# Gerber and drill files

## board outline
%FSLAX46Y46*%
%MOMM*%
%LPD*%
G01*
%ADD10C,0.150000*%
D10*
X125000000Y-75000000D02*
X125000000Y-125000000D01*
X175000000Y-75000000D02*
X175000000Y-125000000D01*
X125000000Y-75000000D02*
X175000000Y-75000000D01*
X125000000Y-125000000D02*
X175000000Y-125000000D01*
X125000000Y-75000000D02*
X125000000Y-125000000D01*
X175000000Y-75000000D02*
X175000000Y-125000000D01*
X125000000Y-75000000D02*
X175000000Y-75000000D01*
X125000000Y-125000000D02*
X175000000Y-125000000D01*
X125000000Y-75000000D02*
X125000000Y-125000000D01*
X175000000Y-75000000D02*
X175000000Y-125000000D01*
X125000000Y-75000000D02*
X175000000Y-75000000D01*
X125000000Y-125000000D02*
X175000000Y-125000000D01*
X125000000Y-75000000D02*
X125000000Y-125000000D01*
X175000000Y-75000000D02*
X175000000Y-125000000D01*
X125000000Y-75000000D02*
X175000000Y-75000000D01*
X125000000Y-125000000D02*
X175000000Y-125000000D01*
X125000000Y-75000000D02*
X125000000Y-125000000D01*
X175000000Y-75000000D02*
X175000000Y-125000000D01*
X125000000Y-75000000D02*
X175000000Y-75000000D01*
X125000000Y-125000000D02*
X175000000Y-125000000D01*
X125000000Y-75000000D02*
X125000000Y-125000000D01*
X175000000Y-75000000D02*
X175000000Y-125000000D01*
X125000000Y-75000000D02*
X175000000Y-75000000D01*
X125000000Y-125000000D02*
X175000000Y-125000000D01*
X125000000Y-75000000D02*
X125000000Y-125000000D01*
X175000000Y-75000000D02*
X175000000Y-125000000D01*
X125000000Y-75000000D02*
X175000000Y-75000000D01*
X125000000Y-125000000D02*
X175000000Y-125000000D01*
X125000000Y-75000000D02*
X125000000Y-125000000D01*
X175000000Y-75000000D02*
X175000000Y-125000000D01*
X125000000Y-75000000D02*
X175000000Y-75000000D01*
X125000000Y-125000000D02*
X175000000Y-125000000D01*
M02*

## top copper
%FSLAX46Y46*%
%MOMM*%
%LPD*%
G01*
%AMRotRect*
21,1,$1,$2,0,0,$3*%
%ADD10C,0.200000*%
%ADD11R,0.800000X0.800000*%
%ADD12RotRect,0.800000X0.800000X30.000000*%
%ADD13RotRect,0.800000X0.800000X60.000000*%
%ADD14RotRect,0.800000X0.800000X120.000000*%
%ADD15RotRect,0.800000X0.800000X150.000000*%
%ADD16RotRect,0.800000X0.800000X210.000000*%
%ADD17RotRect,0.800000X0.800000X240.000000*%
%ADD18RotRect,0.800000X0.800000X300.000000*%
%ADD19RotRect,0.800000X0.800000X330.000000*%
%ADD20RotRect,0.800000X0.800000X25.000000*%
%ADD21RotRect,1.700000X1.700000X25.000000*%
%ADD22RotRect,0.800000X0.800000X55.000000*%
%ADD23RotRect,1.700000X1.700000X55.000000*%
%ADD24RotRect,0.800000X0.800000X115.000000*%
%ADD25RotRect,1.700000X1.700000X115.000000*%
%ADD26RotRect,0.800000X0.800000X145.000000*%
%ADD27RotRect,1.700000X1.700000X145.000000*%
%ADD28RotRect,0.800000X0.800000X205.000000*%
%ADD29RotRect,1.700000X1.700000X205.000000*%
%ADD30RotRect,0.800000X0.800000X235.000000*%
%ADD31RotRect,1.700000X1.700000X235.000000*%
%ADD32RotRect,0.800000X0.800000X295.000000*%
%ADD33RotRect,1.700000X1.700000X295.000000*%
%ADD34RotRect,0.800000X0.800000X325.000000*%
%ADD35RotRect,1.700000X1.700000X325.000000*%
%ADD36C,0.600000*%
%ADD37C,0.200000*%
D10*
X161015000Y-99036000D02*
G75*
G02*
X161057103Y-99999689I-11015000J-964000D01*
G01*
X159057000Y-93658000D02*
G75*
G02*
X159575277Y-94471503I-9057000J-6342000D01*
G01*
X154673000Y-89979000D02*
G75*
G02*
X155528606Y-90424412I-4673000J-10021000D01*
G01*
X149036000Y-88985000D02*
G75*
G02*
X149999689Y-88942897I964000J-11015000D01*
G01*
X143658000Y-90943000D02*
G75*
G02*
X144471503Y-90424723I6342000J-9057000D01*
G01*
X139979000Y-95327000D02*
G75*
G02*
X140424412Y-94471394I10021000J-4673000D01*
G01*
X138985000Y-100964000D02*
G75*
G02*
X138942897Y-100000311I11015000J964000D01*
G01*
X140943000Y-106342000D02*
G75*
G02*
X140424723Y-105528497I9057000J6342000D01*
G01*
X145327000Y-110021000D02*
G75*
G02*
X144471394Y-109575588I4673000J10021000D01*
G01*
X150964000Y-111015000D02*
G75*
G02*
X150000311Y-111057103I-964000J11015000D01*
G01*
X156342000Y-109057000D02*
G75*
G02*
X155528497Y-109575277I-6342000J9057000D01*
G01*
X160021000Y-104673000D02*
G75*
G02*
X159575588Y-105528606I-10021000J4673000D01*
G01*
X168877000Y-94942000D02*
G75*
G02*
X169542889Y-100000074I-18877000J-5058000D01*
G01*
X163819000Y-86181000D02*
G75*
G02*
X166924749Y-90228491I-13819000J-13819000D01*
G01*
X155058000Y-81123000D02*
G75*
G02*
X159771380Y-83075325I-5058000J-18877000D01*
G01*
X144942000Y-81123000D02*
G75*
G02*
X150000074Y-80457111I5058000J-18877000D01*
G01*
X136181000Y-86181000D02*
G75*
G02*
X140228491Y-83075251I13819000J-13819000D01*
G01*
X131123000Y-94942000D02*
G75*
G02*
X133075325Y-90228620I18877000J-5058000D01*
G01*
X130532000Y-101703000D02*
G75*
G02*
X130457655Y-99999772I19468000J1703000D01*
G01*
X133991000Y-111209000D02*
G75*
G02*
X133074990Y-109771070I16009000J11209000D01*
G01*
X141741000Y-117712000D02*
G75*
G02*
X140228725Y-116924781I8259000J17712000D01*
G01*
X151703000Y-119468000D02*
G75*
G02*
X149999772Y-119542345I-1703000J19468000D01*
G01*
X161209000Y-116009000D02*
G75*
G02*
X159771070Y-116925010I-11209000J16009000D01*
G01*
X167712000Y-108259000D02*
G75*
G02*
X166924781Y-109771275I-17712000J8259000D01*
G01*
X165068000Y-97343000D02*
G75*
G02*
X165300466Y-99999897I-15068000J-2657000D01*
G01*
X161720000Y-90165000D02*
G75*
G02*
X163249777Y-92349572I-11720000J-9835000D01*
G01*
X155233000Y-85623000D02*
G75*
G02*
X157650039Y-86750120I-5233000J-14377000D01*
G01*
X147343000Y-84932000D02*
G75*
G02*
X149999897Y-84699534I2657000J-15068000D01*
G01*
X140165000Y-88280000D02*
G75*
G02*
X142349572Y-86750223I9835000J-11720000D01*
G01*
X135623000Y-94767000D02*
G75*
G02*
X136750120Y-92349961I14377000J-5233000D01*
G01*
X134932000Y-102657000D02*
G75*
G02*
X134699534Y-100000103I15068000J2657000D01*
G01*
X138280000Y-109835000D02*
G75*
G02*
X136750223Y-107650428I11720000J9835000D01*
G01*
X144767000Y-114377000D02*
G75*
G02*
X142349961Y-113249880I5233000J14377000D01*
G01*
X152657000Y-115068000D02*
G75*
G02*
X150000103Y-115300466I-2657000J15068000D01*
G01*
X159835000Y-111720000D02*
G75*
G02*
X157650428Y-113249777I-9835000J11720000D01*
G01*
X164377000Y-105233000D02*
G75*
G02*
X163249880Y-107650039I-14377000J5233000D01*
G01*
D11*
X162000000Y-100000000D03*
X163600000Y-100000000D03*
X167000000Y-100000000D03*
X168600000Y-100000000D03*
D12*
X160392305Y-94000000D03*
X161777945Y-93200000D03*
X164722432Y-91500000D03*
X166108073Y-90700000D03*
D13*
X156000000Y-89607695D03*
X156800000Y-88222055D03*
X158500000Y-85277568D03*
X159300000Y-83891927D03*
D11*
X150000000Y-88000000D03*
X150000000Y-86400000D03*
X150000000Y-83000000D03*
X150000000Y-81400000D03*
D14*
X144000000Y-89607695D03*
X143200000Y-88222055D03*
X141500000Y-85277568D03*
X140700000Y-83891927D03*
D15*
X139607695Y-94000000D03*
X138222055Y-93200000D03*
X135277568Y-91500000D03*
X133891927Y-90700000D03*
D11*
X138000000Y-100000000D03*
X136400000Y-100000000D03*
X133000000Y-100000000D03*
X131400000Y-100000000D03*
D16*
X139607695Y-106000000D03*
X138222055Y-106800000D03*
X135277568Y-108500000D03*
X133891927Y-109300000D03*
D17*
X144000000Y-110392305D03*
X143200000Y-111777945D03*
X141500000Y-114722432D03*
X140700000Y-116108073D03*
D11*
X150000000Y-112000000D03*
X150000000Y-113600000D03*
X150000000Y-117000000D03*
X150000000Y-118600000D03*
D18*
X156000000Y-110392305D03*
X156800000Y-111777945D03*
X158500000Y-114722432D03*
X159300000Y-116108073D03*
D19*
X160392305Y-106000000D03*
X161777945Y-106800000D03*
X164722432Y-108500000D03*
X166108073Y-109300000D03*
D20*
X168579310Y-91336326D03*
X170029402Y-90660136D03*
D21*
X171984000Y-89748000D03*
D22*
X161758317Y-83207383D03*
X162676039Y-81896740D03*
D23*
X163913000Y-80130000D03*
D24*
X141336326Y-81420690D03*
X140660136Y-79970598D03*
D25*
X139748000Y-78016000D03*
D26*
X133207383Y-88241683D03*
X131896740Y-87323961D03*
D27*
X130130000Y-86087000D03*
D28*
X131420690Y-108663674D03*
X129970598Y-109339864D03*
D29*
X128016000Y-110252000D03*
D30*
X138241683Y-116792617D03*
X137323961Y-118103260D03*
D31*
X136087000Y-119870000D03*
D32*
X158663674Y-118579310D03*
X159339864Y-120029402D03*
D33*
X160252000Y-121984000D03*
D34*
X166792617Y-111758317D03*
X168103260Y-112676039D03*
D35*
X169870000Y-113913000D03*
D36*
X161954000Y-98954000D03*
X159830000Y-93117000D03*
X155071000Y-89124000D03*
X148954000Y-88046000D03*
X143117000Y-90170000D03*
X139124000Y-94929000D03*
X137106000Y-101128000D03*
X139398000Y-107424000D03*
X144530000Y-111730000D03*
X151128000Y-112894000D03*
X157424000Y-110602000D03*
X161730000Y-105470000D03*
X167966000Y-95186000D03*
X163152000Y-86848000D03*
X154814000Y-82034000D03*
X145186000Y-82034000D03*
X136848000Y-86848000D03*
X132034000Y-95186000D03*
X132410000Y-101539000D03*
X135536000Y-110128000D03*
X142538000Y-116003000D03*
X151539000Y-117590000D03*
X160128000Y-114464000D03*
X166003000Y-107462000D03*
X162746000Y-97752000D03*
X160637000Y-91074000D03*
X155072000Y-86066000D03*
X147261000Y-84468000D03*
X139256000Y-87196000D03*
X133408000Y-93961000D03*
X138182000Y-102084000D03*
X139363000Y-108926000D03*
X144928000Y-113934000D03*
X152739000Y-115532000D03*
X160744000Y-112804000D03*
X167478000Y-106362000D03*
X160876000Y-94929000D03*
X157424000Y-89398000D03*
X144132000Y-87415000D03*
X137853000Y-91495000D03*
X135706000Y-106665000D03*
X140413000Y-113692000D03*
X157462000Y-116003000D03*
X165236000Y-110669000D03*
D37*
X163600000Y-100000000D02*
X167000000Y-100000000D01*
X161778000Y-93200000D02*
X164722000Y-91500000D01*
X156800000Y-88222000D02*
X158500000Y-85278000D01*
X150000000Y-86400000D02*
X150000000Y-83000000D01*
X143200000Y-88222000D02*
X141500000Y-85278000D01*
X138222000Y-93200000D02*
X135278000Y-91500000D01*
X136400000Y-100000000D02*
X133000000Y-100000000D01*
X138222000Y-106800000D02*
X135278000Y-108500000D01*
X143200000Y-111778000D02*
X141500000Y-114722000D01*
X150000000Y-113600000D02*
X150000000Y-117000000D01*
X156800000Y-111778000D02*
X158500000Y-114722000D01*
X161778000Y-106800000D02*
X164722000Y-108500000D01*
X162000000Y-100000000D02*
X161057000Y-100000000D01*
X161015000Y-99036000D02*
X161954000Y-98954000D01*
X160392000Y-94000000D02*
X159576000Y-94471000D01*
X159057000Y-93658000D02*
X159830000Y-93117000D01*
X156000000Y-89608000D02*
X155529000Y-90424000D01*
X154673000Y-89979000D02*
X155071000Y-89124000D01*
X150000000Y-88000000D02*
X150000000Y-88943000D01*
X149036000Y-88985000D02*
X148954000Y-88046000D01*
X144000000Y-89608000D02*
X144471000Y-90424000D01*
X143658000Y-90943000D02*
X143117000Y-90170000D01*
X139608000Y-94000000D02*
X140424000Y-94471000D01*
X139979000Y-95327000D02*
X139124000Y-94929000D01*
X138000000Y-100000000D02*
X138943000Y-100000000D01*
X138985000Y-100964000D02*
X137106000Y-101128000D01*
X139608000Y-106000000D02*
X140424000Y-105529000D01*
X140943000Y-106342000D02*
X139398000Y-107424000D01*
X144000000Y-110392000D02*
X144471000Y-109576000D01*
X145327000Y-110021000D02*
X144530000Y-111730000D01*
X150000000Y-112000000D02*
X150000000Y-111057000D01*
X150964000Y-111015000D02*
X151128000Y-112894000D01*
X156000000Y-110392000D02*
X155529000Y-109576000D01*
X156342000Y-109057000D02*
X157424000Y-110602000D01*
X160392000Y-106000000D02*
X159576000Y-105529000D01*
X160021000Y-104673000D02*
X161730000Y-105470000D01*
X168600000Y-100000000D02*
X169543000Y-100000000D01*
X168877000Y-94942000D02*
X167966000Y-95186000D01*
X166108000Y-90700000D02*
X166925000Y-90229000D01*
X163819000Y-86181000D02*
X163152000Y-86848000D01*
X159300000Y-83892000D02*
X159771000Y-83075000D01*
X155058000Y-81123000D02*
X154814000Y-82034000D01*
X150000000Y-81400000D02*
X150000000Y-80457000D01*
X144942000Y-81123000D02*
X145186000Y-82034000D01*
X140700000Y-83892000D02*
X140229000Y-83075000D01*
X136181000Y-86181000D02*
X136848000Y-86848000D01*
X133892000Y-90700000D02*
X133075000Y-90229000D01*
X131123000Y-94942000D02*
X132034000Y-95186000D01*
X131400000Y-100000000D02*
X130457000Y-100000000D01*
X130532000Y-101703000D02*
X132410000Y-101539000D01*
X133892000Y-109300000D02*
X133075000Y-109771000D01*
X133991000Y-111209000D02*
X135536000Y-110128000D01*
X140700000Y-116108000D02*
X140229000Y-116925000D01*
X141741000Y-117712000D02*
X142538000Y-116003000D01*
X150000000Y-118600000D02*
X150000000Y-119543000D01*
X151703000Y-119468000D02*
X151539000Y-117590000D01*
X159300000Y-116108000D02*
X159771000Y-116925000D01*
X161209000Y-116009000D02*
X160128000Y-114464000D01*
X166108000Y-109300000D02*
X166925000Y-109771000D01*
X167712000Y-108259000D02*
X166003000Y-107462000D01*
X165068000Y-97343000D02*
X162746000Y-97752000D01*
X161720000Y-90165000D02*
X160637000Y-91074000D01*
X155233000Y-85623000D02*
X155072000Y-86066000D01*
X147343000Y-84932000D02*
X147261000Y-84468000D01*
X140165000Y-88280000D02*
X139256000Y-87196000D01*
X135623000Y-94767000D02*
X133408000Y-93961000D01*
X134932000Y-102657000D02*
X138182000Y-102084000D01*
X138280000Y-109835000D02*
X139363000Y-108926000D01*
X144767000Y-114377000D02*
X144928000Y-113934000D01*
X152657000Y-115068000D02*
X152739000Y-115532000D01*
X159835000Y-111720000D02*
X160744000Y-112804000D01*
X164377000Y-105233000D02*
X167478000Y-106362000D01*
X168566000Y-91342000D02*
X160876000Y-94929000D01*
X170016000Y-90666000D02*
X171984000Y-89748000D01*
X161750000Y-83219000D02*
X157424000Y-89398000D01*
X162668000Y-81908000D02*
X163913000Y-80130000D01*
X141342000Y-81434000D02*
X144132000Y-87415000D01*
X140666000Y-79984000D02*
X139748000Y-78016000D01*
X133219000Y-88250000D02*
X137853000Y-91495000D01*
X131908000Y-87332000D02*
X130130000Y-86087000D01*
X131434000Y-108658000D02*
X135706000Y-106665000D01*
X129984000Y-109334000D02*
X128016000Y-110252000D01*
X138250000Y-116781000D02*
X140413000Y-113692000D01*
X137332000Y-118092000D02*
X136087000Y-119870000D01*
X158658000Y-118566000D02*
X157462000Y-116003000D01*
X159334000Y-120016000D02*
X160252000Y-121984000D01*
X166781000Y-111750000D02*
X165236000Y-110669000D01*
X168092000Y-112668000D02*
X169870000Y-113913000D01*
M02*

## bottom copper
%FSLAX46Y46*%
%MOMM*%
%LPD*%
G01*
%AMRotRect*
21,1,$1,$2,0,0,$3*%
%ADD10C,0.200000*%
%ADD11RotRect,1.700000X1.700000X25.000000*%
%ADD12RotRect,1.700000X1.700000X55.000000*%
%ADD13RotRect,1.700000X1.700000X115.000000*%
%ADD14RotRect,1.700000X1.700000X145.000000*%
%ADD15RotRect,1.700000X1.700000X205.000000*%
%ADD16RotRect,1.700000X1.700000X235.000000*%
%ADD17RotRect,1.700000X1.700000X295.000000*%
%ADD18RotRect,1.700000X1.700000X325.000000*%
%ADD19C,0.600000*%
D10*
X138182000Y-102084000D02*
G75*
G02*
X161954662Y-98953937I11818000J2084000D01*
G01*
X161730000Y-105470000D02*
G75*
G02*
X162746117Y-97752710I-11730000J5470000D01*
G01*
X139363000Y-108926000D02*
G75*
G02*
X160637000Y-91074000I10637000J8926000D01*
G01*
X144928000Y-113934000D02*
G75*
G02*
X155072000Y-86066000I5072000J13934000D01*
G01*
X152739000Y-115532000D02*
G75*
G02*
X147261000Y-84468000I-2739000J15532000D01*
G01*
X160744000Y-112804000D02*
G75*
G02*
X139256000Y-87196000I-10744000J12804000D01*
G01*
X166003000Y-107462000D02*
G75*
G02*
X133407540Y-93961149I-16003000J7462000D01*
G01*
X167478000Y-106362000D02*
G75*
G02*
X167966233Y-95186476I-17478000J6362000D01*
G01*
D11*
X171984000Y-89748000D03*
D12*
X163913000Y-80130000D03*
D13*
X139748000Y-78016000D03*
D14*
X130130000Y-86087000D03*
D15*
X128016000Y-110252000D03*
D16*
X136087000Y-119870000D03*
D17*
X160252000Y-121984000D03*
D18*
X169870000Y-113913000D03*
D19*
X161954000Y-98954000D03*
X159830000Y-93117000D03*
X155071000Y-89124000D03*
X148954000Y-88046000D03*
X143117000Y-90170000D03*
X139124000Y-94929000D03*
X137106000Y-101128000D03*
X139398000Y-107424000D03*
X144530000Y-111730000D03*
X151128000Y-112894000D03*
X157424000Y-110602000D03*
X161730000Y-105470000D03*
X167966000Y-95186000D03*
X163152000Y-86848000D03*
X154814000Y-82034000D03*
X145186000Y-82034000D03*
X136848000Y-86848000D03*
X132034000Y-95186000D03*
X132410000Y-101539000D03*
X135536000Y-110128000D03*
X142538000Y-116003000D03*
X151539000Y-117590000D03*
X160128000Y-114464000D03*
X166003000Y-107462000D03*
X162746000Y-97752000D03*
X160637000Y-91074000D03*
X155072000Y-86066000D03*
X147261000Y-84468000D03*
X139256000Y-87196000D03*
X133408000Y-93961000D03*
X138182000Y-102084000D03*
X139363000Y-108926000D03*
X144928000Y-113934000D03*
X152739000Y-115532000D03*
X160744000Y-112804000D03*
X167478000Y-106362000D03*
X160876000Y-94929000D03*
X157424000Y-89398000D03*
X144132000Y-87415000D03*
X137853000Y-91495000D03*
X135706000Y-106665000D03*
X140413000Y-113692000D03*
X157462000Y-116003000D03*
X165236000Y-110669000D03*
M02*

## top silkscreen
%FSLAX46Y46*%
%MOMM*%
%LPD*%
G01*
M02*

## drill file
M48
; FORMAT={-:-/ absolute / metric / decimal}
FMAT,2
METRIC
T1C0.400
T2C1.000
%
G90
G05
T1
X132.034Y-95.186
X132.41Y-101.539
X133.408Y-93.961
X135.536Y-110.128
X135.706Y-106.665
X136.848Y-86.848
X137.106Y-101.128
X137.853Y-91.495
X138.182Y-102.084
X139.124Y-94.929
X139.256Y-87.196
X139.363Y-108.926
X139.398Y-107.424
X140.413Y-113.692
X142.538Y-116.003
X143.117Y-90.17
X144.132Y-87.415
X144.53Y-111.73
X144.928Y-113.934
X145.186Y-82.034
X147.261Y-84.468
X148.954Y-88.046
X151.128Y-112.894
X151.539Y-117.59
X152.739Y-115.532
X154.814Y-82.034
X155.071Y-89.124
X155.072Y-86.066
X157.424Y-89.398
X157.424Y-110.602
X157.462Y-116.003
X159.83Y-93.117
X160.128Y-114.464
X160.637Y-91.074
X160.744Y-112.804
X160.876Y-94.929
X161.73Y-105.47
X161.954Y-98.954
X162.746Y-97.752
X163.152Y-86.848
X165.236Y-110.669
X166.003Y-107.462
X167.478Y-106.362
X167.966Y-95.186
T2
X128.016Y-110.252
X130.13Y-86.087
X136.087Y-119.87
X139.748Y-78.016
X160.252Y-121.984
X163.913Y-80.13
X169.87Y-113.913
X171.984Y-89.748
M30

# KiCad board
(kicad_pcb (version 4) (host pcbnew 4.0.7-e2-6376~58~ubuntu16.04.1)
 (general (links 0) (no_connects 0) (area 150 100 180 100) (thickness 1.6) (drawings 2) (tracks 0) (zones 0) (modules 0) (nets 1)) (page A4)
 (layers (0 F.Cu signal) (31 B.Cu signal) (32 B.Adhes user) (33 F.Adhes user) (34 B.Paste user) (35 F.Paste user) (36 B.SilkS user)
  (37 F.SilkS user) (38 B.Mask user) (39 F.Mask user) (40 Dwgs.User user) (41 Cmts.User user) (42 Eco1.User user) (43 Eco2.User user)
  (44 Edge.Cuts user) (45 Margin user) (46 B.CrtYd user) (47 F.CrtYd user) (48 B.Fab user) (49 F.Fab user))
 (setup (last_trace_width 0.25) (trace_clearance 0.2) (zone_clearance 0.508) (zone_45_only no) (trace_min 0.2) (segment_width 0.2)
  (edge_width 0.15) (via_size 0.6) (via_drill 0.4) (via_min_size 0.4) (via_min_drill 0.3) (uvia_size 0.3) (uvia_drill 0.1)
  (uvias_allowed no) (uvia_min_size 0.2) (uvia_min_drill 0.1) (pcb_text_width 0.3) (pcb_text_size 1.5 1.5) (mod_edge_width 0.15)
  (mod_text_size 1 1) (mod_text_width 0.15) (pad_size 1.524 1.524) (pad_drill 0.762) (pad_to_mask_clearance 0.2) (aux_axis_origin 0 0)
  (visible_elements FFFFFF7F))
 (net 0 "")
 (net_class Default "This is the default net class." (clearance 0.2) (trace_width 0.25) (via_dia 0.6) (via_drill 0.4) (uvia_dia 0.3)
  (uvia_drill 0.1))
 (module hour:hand (layer F.Cu) (at 150 100 0.0)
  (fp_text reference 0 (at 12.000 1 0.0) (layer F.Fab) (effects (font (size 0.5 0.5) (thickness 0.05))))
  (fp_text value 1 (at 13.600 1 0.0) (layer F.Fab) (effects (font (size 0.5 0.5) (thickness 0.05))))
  (pad 1 smd rect (at 12.0 0 0.0) (size 0.8 0.8) (layers F.Cu F.Paste F.Mask))
  (pad 2 smd rect (at 13.6 0 0.0) (size 0.8 0.8) (layers F.Cu F.Paste F.Mask)))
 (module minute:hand (layer F.Cu) (at 150 100 0.0)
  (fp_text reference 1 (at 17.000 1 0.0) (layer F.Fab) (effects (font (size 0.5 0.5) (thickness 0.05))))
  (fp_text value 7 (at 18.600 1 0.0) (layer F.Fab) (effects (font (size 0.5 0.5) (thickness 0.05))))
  (pad 1 smd rect (at 17.0 0 0.0) (size 0.8 0.8) (layers F.Cu F.Paste F.Mask))
  (pad 2 smd rect (at 18.6 0 0.0) (size 0.8 0.8) (layers F.Cu F.Paste F.Mask)))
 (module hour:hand (layer F.Cu) (at 150 100 30.0)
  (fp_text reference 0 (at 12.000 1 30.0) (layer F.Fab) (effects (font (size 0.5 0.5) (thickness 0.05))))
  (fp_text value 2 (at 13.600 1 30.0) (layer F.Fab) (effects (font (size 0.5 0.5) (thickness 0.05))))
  (pad 1 smd rect (at 12.0 0 30.0) (size 0.8 0.8) (layers F.Cu F.Paste F.Mask))
  (pad 2 smd rect (at 13.6 0 30.0) (size 0.8 0.8) (layers F.Cu F.Paste F.Mask)))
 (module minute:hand (layer F.Cu) (at 150 100 30.0)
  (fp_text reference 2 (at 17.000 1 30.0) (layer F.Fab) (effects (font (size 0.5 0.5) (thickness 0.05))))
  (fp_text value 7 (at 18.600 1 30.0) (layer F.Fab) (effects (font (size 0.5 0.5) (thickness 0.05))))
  (pad 1 smd rect (at 17.0 0 30.0) (size 0.8 0.8) (layers F.Cu F.Paste F.Mask))
  (pad 2 smd rect (at 18.6 0 30.0) (size 0.8 0.8) (layers F.Cu F.Paste F.Mask)))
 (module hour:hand (layer F.Cu) (at 150 100 60.0)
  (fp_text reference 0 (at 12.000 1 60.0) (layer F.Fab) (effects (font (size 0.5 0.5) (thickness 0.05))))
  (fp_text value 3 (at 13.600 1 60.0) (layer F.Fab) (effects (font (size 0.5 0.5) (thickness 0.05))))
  (pad 1 smd rect (at 12.0 0 60.0) (size 0.8 0.8) (layers F.Cu F.Paste F.Mask))
  (pad 2 smd rect (at 13.6 0 60.0) (size 0.8 0.8) (layers F.Cu F.Paste F.Mask)))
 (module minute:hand (layer F.Cu) (at 150 100 60.0)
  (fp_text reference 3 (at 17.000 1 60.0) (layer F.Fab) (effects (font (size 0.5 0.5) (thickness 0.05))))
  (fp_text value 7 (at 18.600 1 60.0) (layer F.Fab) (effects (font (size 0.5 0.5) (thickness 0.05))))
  (pad 1 smd rect (at 17.0 0 60.0) (size 0.8 0.8) (layers F.Cu F.Paste F.Mask))
  (pad 2 smd rect (at 18.6 0 60.0) (size 0.8 0.8) (layers F.Cu F.Paste F.Mask)))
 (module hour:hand (layer F.Cu) (at 150 100 90.0)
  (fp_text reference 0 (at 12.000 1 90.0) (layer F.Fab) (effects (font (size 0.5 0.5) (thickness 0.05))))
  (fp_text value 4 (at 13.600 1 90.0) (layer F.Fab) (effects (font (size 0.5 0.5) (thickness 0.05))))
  (pad 1 smd rect (at 12.0 0 90.0) (size 0.8 0.8) (layers F.Cu F.Paste F.Mask))
  (pad 2 smd rect (at 13.6 0 90.0) (size 0.8 0.8) (layers F.Cu F.Paste F.Mask)))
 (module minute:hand (layer F.Cu) (at 150 100 90.0)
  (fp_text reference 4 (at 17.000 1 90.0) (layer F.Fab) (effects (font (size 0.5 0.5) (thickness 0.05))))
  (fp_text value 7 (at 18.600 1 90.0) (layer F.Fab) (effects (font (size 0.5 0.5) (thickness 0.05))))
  (pad 1 smd rect (at 17.0 0 90.0) (size 0.8 0.8) (layers F.Cu F.Paste F.Mask))
  (pad 2 smd rect (at 18.6 0 90.0) (size 0.8 0.8) (layers F.Cu F.Paste F.Mask)))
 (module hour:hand (layer F.Cu) (at 150 100 120.0)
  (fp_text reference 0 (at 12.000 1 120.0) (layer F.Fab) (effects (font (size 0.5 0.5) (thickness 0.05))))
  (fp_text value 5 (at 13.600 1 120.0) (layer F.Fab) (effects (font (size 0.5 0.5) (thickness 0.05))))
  (pad 1 smd rect (at 12.0 0 120.0) (size 0.8 0.8) (layers F.Cu F.Paste F.Mask))
  (pad 2 smd rect (at 13.6 0 120.0) (size 0.8 0.8) (layers F.Cu F.Paste F.Mask)))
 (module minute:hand (layer F.Cu) (at 150 100 120.0)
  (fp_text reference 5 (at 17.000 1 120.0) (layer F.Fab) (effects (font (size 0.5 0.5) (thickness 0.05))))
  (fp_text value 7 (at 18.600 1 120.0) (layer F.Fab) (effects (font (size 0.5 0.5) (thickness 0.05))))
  (pad 1 smd rect (at 17.0 0 120.0) (size 0.8 0.8) (layers F.Cu F.Paste F.Mask))
  (pad 2 smd rect (at 18.6 0 120.0) (size 0.8 0.8) (layers F.Cu F.Paste F.Mask)))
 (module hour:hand (layer F.Cu) (at 150 100 150.0)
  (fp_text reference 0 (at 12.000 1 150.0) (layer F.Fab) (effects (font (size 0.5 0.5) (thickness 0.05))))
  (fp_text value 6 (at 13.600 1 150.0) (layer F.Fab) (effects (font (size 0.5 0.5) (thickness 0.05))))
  (pad 1 smd rect (at 12.0 0 150.0) (size 0.8 0.8) (layers F.Cu F.Paste F.Mask))
  (pad 2 smd rect (at 13.6 0 150.0) (size 0.8 0.8) (layers F.Cu F.Paste F.Mask)))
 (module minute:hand (layer F.Cu) (at 150 100 150.0)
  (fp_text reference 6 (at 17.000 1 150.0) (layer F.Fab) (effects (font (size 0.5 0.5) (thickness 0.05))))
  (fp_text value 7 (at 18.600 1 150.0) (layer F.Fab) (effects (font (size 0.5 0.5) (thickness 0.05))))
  (pad 1 smd rect (at 17.0 0 150.0) (size 0.8 0.8) (layers F.Cu F.Paste F.Mask))
  (pad 2 smd rect (at 18.6 0 150.0) (size 0.8 0.8) (layers F.Cu F.Paste F.Mask)))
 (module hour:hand (layer F.Cu) (at 150 100 180.0)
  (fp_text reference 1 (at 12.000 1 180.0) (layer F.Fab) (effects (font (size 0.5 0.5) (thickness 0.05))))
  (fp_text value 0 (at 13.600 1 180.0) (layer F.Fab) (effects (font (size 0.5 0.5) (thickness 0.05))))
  (pad 1 smd rect (at 12.0 0 180.0) (size 0.8 0.8) (layers F.Cu F.Paste F.Mask))
  (pad 2 smd rect (at 13.6 0 180.0) (size 0.8 0.8) (layers F.Cu F.Paste F.Mask)))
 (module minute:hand (layer F.Cu) (at 150 100 180.0)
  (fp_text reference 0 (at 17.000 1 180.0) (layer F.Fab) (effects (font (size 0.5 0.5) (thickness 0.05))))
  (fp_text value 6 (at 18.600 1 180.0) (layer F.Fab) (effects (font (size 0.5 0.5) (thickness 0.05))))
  (pad 1 smd rect (at 17.0 0 180.0) (size 0.8 0.8) (layers F.Cu F.Paste F.Mask))
  (pad 2 smd rect (at 18.6 0 180.0) (size 0.8 0.8) (layers F.Cu F.Paste F.Mask)))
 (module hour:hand (layer F.Cu) (at 150 100 210.0)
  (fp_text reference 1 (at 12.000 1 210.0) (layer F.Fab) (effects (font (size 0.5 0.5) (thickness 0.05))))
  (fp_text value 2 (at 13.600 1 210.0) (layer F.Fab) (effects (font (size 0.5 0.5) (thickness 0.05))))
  (pad 1 smd rect (at 12.0 0 210.0) (size 0.8 0.8) (layers F.Cu F.Paste F.Mask))
  (pad 2 smd rect (at 13.6 0 210.0) (size 0.8 0.8) (layers F.Cu F.Paste F.Mask)))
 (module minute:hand (layer F.Cu) (at 150 100 210.0)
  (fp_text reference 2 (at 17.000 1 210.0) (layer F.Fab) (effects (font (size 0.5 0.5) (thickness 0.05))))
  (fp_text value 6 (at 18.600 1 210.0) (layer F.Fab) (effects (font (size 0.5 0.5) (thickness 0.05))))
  (pad 1 smd rect (at 17.0 0 210.0) (size 0.8 0.8) (layers F.Cu F.Paste F.Mask))
  (pad 2 smd rect (at 18.6 0 210.0) (size 0.8 0.8) (layers F.Cu F.Paste F.Mask)))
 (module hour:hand (layer F.Cu) (at 150 100 240.0)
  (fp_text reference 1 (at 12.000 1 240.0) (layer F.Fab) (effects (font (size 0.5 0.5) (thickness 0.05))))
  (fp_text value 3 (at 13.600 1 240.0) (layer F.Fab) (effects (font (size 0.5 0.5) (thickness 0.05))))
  (pad 1 smd rect (at 12.0 0 240.0) (size 0.8 0.8) (layers F.Cu F.Paste F.Mask))
  (pad 2 smd rect (at 13.6 0 240.0) (size 0.8 0.8) (layers F.Cu F.Paste F.Mask)))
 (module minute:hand (layer F.Cu) (at 150 100 240.0)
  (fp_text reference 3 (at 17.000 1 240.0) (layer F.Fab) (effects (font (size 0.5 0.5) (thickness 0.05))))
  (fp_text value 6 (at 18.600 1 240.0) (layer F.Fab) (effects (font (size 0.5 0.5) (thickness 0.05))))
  (pad 1 smd rect (at 17.0 0 240.0) (size 0.8 0.8) (layers F.Cu F.Paste F.Mask))
  (pad 2 smd rect (at 18.6 0 240.0) (size 0.8 0.8) (layers F.Cu F.Paste F.Mask)))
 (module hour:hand (layer F.Cu) (at 150 100 270.0)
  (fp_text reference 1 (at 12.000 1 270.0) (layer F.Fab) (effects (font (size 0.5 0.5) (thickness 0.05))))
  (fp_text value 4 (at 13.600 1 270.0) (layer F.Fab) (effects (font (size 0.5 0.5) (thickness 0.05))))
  (pad 1 smd rect (at 12.0 0 270.0) (size 0.8 0.8) (layers F.Cu F.Paste F.Mask))
  (pad 2 smd rect (at 13.6 0 270.0) (size 0.8 0.8) (layers F.Cu F.Paste F.Mask)))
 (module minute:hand (layer F.Cu) (at 150 100 270.0)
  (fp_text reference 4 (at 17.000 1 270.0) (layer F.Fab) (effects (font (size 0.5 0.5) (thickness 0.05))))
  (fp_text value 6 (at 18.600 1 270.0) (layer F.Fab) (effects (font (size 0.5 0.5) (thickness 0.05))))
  (pad 1 smd rect (at 17.0 0 270.0) (size 0.8 0.8) (layers F.Cu F.Paste F.Mask))
  (pad 2 smd rect (at 18.6 0 270.0) (size 0.8 0.8) (layers F.Cu F.Paste F.Mask)))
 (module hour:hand (layer F.Cu) (at 150 100 300.0)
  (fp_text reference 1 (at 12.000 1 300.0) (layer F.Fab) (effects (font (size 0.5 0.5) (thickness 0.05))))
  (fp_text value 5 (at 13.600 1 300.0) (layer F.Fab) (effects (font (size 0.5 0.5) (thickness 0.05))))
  (pad 1 smd rect (at 12.0 0 300.0) (size 0.8 0.8) (layers F.Cu F.Paste F.Mask))
  (pad 2 smd rect (at 13.6 0 300.0) (size 0.8 0.8) (layers F.Cu F.Paste F.Mask)))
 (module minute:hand (layer F.Cu) (at 150 100 300.0)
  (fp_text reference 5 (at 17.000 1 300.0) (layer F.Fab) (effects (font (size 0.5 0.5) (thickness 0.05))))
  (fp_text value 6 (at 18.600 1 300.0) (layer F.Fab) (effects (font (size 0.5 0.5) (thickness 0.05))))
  (pad 1 smd rect (at 17.0 0 300.0) (size 0.8 0.8) (layers F.Cu F.Paste F.Mask))
  (pad 2 smd rect (at 18.6 0 300.0) (size 0.8 0.8) (layers F.Cu F.Paste F.Mask)))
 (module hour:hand (layer F.Cu) (at 150 100 330.0)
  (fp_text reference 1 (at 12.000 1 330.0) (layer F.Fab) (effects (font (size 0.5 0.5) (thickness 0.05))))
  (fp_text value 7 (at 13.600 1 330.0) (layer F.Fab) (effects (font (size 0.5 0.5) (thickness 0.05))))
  (pad 1 smd rect (at 12.0 0 330.0) (size 0.8 0.8) (layers F.Cu F.Paste F.Mask))
  (pad 2 smd rect (at 13.6 0 330.0) (size 0.8 0.8) (layers F.Cu F.Paste F.Mask)))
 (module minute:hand (layer F.Cu) (at 150 100 330.0)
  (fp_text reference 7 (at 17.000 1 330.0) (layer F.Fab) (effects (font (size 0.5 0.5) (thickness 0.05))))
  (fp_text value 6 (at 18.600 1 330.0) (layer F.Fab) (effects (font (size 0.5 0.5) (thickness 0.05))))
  (pad 1 smd rect (at 17.0 0 330.0) (size 0.8 0.8) (layers F.Cu F.Paste F.Mask))
  (pad 2 smd rect (at 18.6 0 330.0) (size 0.8 0.8) (layers F.Cu F.Paste F.Mask)))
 (segment (start 163.600 100.000) (end 167.000 100.000) (width 0.2) (layer F.Cu) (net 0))
 (segment (start 161.778 93.200) (end 164.722 91.500) (width 0.2) (layer F.Cu) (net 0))
 (segment (start 156.800 88.222) (end 158.500 85.278) (width 0.2) (layer F.Cu) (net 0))
 (segment (start 150.000 86.400) (end 150.000 83.000) (width 0.2) (layer F.Cu) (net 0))
 (segment (start 143.200 88.222) (end 141.500 85.278) (width 0.2) (layer F.Cu) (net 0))
 (segment (start 138.222 93.200) (end 135.278 91.500) (width 0.2) (layer F.Cu) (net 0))
 (segment (start 136.400 100.000) (end 133.000 100.000) (width 0.2) (layer F.Cu) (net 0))
 (segment (start 138.222 106.800) (end 135.278 108.500) (width 0.2) (layer F.Cu) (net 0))
 (segment (start 143.200 111.778) (end 141.500 114.722) (width 0.2) (layer F.Cu) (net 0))
 (segment (start 150.000 113.600) (end 150.000 117.000) (width 0.2) (layer F.Cu) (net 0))
 (segment (start 156.800 111.778) (end 158.500 114.722) (width 0.2) (layer F.Cu) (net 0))
 (segment (start 161.778 106.800) (end 164.722 108.500) (width 0.2) (layer F.Cu) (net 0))
 (gr_arc (start 150 100) (end 138.182 102.084) (angle 185.000) (layer B.Cu) (width 0.2))
 (gr_arc (start 150 100) (end 161.730 105.470) (angle 325.000) (layer B.Cu) (width 0.2))
 (gr_arc (start 150 100) (end 139.363 108.926) (angle 180.000) (layer B.Cu) (width 0.2))
 (gr_arc (start 150 100) (end 144.928 113.934) (angle 180.000) (layer B.Cu) (width 0.2))
 (gr_arc (start 150 100) (end 152.739 115.532) (angle 180.000) (layer B.Cu) (width 0.2))
 (gr_arc (start 150 100) (end 160.744 112.804) (angle 180.000) (layer B.Cu) (width 0.2))
 (gr_arc (start 150 100) (end 166.003 107.462) (angle 175.000) (layer B.Cu) (width 0.2))
 (gr_arc (start 150 100) (end 167.478 106.362) (angle 325.000) (layer B.Cu) (width 0.2))
 (segment (start 162.000 100.000) (end 161.057 100.000) (width 0.2) (layer F.Cu) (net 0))
 (gr_arc (start 150 100) (end 161.015 99.036) (angle 5.000) (layer F.Cu) (width 0.2))
 (segment (start 161.015 99.036) (end 161.954 98.954) (width 0.2) (layer F.Cu) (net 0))
 (via (at 161.954 98.954) (size 0.6) (drill 0.4) (layers F.Cu B.Cu) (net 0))
 (segment (start 160.392 94.000) (end 159.576 94.471) (width 0.2) (layer F.Cu) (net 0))
 (gr_arc (start 150 100) (end 159.057 93.658) (angle 5.000) (layer F.Cu) (width 0.2))
 (segment (start 159.057 93.658) (end 159.830 93.117) (width 0.2) (layer F.Cu) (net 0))
 (via (at 159.830 93.117) (size 0.6) (drill 0.4) (layers F.Cu B.Cu) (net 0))
 (segment (start 156.000 89.608) (end 155.529 90.424) (width 0.2) (layer F.Cu) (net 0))
 (gr_arc (start 150 100) (end 154.673 89.979) (angle 5.000) (layer F.Cu) (width 0.2))
 (segment (start 154.673 89.979) (end 155.071 89.124) (width 0.2) (layer F.Cu) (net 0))
 (via (at 155.071 89.124) (size 0.6) (drill 0.4) (layers F.Cu B.Cu) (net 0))
 (segment (start 150.000 88.000) (end 150.000 88.943) (width 0.2) (layer F.Cu) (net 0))
 (gr_arc (start 150 100) (end 149.036 88.985) (angle 5.000) (layer F.Cu) (width 0.2))
 (segment (start 149.036 88.985) (end 148.954 88.046) (width 0.2) (layer F.Cu) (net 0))
 (via (at 148.954 88.046) (size 0.6) (drill 0.4) (layers F.Cu B.Cu) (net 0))
 (segment (start 144.000 89.608) (end 144.471 90.424) (width 0.2) (layer F.Cu) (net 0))
 (gr_arc (start 150 100) (end 143.658 90.943) (angle 5.000) (layer F.Cu) (width 0.2))
 (segment (start 143.658 90.943) (end 143.117 90.170) (width 0.2) (layer F.Cu) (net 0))
 (via (at 143.117 90.170) (size 0.6) (drill 0.4) (layers F.Cu B.Cu) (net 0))
 (segment (start 139.608 94.000) (end 140.424 94.471) (width 0.2) (layer F.Cu) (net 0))
 (gr_arc (start 150 100) (end 139.979 95.327) (angle 5.000) (layer F.Cu) (width 0.2))
 (segment (start 139.979 95.327) (end 139.124 94.929) (width 0.2) (layer F.Cu) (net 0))
 (via (at 139.124 94.929) (size 0.6) (drill 0.4) (layers F.Cu B.Cu) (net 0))
 (segment (start 138.000 100.000) (end 138.943 100.000) (width 0.2) (layer F.Cu) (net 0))
 (gr_arc (start 150 100) (end 138.985 100.964) (angle 5.000) (layer F.Cu) (width 0.2))
 (segment (start 138.985 100.964) (end 137.106 101.128) (width 0.2) (layer F.Cu) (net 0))
 (via (at 137.106 101.128) (size 0.6) (drill 0.4) (layers F.Cu B.Cu) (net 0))
 (segment (start 139.608 106.000) (end 140.424 105.529) (width 0.2) (layer F.Cu) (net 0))
 (gr_arc (start 150 100) (end 140.943 106.342) (angle 5.000) (layer F.Cu) (width 0.2))
 (segment (start 140.943 106.342) (end 139.398 107.424) (width 0.2) (layer F.Cu) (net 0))
 (via (at 139.398 107.424) (size 0.6) (drill 0.4) (layers F.Cu B.Cu) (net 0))
 (segment (start 144.000 110.392) (end 144.471 109.576) (width 0.2) (layer F.Cu) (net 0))
 (gr_arc (start 150 100) (end 145.327 110.021) (angle 5.000) (layer F.Cu) (width 0.2))
 (segment (start 145.327 110.021) (end 144.530 111.730) (width 0.2) (layer F.Cu) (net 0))
 (via (at 144.530 111.730) (size 0.6) (drill 0.4) (layers F.Cu B.Cu) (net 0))
 (segment (start 150.000 112.000) (end 150.000 111.057) (width 0.2) (layer F.Cu) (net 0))
 (gr_arc (start 150 100) (end 150.964 111.015) (angle 5.000) (layer F.Cu) (width 0.2))
 (segment (start 150.964 111.015) (end 151.128 112.894) (width 0.2) (layer F.Cu) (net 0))
 (via (at 151.128 112.894) (size 0.6) (drill 0.4) (layers F.Cu B.Cu) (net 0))
 (segment (start 156.000 110.392) (end 155.529 109.576) (width 0.2) (layer F.Cu) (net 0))
 (gr_arc (start 150 100) (end 156.342 109.057) (angle 5.000) (layer F.Cu) (width 0.2))
 (segment (start 156.342 109.057) (end 157.424 110.602) (width 0.2) (layer F.Cu) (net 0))
 (via (at 157.424 110.602) (size 0.6) (drill 0.4) (layers F.Cu B.Cu) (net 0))
 (segment (start 160.392 106.000) (end 159.576 105.529) (width 0.2) (layer F.Cu) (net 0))
 (gr_arc (start 150 100) (end 160.021 104.673) (angle 5.000) (layer F.Cu) (width 0.2))
 (segment (start 160.021 104.673) (end 161.730 105.470) (width 0.2) (layer F.Cu) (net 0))
 (via (at 161.730 105.470) (size 0.6) (drill 0.4) (layers F.Cu B.Cu) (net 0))
 (segment (start 168.600 100.000) (end 169.543 100.000) (width 0.2) (layer F.Cu) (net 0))
 (gr_arc (start 150 100) (end 168.877 94.942) (angle 15.000) (layer F.Cu) (width 0.2))
 (segment (start 168.877 94.942) (end 167.966 95.186) (width 0.2) (layer F.Cu) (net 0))
 (via (at 167.966 95.186) (size 0.6) (drill 0.4) (layers F.Cu B.Cu) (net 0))
 (segment (start 166.108 90.700) (end 166.925 90.229) (width 0.2) (layer F.Cu) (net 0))
 (gr_arc (start 150 100) (end 163.819 86.181) (angle 15.000) (layer F.Cu) (width 0.2))
 (segment (start 163.819 86.181) (end 163.152 86.848) (width 0.2) (layer F.Cu) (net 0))
 (via (at 163.152 86.848) (size 0.6) (drill 0.4) (layers F.Cu B.Cu) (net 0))
 (segment (start 159.300 83.892) (end 159.771 83.075) (width 0.2) (layer F.Cu) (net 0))
 (gr_arc (start 150 100) (end 155.058 81.123) (angle 15.000) (layer F.Cu) (width 0.2))
 (segment (start 155.058 81.123) (end 154.814 82.034) (width 0.2) (layer F.Cu) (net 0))
 (via (at 154.814 82.034) (size 0.6) (drill 0.4) (layers F.Cu B.Cu) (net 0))
 (segment (start 150.000 81.400) (end 150.000 80.457) (width 0.2) (layer F.Cu) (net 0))
 (gr_arc (start 150 100) (end 144.942 81.123) (angle 15.000) (layer F.Cu) (width 0.2))
 (segment (start 144.942 81.123) (end 145.186 82.034) (width 0.2) (layer F.Cu) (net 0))
 (via (at 145.186 82.034) (size 0.6) (drill 0.4) (layers F.Cu B.Cu) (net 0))
 (segment (start 140.700 83.892) (end 140.229 83.075) (width 0.2) (layer F.Cu) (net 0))
 (gr_arc (start 150 100) (end 136.181 86.181) (angle 15.000) (layer F.Cu) (width 0.2))
 (segment (start 136.181 86.181) (end 136.848 86.848) (width 0.2) (layer F.Cu) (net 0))
 (via (at 136.848 86.848) (size 0.6) (drill 0.4) (layers F.Cu B.Cu) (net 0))
 (segment (start 133.892 90.700) (end 133.075 90.229) (width 0.2) (layer F.Cu) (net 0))
 (gr_arc (start 150 100) (end 131.123 94.942) (angle 15.000) (layer F.Cu) (width 0.2))
 (segment (start 131.123 94.942) (end 132.034 95.186) (width 0.2) (layer F.Cu) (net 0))
 (via (at 132.034 95.186) (size 0.6) (drill 0.4) (layers F.Cu B.Cu) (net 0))
 (segment (start 131.400 100.000) (end 130.457 100.000) (width 0.2) (layer F.Cu) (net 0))
 (gr_arc (start 150 100) (end 130.532 101.703) (angle 5.000) (layer F.Cu) (width 0.2))
 (segment (start 130.532 101.703) (end 132.410 101.539) (width 0.2) (layer F.Cu) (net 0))
 (via (at 132.410 101.539) (size 0.6) (drill 0.4) (layers F.Cu B.Cu) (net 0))
 (segment (start 133.892 109.300) (end 133.075 109.771) (width 0.2) (layer F.Cu) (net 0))
 (gr_arc (start 150 100) (end 133.991 111.209) (angle 5.000) (layer F.Cu) (width 0.2))
 (segment (start 133.991 111.209) (end 135.536 110.128) (width 0.2) (layer F.Cu) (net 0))
 (via (at 135.536 110.128) (size 0.6) (drill 0.4) (layers F.Cu B.Cu) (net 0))
 (segment (start 140.700 116.108) (end 140.229 116.925) (width 0.2) (layer F.Cu) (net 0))
 (gr_arc (start 150 100) (end 141.741 117.712) (angle 5.000) (layer F.Cu) (width 0.2))
 (segment (start 141.741 117.712) (end 142.538 116.003) (width 0.2) (layer F.Cu) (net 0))
 (via (at 142.538 116.003) (size 0.6) (drill 0.4) (layers F.Cu B.Cu) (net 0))
 (segment (start 150.000 118.600) (end 150.000 119.543) (width 0.2) (layer F.Cu) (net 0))
 (gr_arc (start 150 100) (end 151.703 119.468) (angle 5.000) (layer F.Cu) (width 0.2))
 (segment (start 151.703 119.468) (end 151.539 117.590) (width 0.2) (layer F.Cu) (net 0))
 (via (at 151.539 117.590) (size 0.6) (drill 0.4) (layers F.Cu B.Cu) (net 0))
 (segment (start 159.300 116.108) (end 159.771 116.925) (width 0.2) (layer F.Cu) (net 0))
 (gr_arc (start 150 100) (end 161.209 116.009) (angle 5.000) (layer F.Cu) (width 0.2))
 (segment (start 161.209 116.009) (end 160.128 114.464) (width 0.2) (layer F.Cu) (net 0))
 (via (at 160.128 114.464) (size 0.6) (drill 0.4) (layers F.Cu B.Cu) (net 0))
 (segment (start 166.108 109.300) (end 166.925 109.771) (width 0.2) (layer F.Cu) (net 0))
 (gr_arc (start 150 100) (end 167.712 108.259) (angle 5.000) (layer F.Cu) (width 0.2))
 (segment (start 167.712 108.259) (end 166.003 107.462) (width 0.2) (layer F.Cu) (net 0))
 (via (at 166.003 107.462) (size 0.6) (drill 0.4) (layers F.Cu B.Cu) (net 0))
 (gr_arc (start 150 100) (end 165.068 97.343) (angle 10.000) (layer F.Cu) (width 0.2))
 (segment (start 165.068 97.343) (end 162.746 97.752) (width 0.2) (layer F.Cu) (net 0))
 (via (at 162.746 97.752) (size 0.6) (drill 0.4) (layers F.Cu B.Cu) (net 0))
 (gr_arc (start 150 100) (end 161.720 90.165) (angle 10.000) (layer F.Cu) (width 0.2))
 (segment (start 161.720 90.165) (end 160.637 91.074) (width 0.2) (layer F.Cu) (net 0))
 (via (at 160.637 91.074) (size 0.6) (drill 0.4) (layers F.Cu B.Cu) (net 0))
 (gr_arc (start 150 100) (end 155.233 85.623) (angle 10.000) (layer F.Cu) (width 0.2))
 (segment (start 155.233 85.623) (end 155.072 86.066) (width 0.2) (layer F.Cu) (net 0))
 (via (at 155.072 86.066) (size 0.6) (drill 0.4) (layers F.Cu B.Cu) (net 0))
 (gr_arc (start 150 100) (end 147.343 84.932) (angle 10.000) (layer F.Cu) (width 0.2))
 (segment (start 147.343 84.932) (end 147.261 84.468) (width 0.2) (layer F.Cu) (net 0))
 (via (at 147.261 84.468) (size 0.6) (drill 0.4) (layers F.Cu B.Cu) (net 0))
 (gr_arc (start 150 100) (end 140.165 88.280) (angle 10.000) (layer F.Cu) (width 0.2))
 (segment (start 140.165 88.280) (end 139.256 87.196) (width 0.2) (layer F.Cu) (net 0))
 (via (at 139.256 87.196) (size 0.6) (drill 0.4) (layers F.Cu B.Cu) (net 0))
 (gr_arc (start 150 100) (end 135.623 94.767) (angle 10.000) (layer F.Cu) (width 0.2))
 (segment (start 135.623 94.767) (end 133.408 93.961) (width 0.2) (layer F.Cu) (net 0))
 (via (at 133.408 93.961) (size 0.6) (drill 0.4) (layers F.Cu B.Cu) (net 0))
 (gr_arc (start 150 100) (end 134.932 102.657) (angle 10.000) (layer F.Cu) (width 0.2))
 (segment (start 134.932 102.657) (end 138.182 102.084) (width 0.2) (layer F.Cu) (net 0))
 (via (at 138.182 102.084) (size 0.6) (drill 0.4) (layers F.Cu B.Cu) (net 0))
 (gr_arc (start 150 100) (end 138.280 109.835) (angle 10.000) (layer F.Cu) (width 0.2))
 (segment (start 138.280 109.835) (end 139.363 108.926) (width 0.2) (layer F.Cu) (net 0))
 (via (at 139.363 108.926) (size 0.6) (drill 0.4) (layers F.Cu B.Cu) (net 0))
 (gr_arc (start 150 100) (end 144.767 114.377) (angle 10.000) (layer F.Cu) (width 0.2))
 (segment (start 144.767 114.377) (end 144.928 113.934) (width 0.2) (layer F.Cu) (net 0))
 (via (at 144.928 113.934) (size 0.6) (drill 0.4) (layers F.Cu B.Cu) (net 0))
 (gr_arc (start 150 100) (end 152.657 115.068) (angle 10.000) (layer F.Cu) (width 0.2))
 (segment (start 152.657 115.068) (end 152.739 115.532) (width 0.2) (layer F.Cu) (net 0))
 (via (at 152.739 115.532) (size 0.6) (drill 0.4) (layers F.Cu B.Cu) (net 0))
 (gr_arc (start 150 100) (end 159.835 111.720) (angle 10.000) (layer F.Cu) (width 0.2))
 (segment (start 159.835 111.720) (end 160.744 112.804) (width 0.2) (layer F.Cu) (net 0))
 (via (at 160.744 112.804) (size 0.6) (drill 0.4) (layers F.Cu B.Cu) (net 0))
 (gr_arc (start 150 100) (end 164.377 105.233) (angle 10.000) (layer F.Cu) (width 0.2))
 (segment (start 164.377 105.233) (end 167.478 106.362) (width 0.2) (layer F.Cu) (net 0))
 (via (at 167.478 106.362) (size 0.6) (drill 0.4) (layers F.Cu B.Cu) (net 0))
 (segment (start 168.566 91.342) (end 160.876 94.929) (width 0.2) (layer F.Cu) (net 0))
 (via (at 160.876 94.929) (size 0.6) (drill 0.4) (layers F.Cu B.Cu) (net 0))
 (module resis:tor (layer F.Cu) (at 150 100 25.0)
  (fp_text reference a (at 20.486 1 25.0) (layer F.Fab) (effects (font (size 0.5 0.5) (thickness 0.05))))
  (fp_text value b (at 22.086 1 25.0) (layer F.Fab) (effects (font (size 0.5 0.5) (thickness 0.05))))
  (pad 1 smd rect (at 20.5 0 25.0) (size 0.8 0.8) (layers F.Cu F.Paste F.Mask))
  (pad 2 smd rect (at 22.1 0 25.0) (size 0.8 0.8) (layers F.Cu F.Paste F.Mask)))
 (segment (start 170.016 90.666) (end 171.984 89.748) (width 0.2) (layer F.Cu) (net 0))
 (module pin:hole (layer F.Cu) (at 171.984 89.748)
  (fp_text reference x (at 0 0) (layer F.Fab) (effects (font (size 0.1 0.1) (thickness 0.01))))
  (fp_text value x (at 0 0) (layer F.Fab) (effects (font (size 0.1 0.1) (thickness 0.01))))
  (pad 0 thru_hole rect (at 0 0 25.0) (size 1.7 1.7) (drill 1) (layers *.Cu *.Mask)))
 (gr_line (start 125.000 75.000) (end 125.000 125.000) (angle 90) (layer Edge.Cuts) (width 0.15))
 (gr_line (start 175.000 75.000) (end 175.000 125.000) (angle 90) (layer Edge.Cuts) (width 0.15))
 (gr_line (start 125.000 75.000) (end 175.000 75.000) (angle 0) (layer Edge.Cuts) (width 0.15))
 (gr_line (start 125.000 125.000) (end 175.000 125.000) (angle 0) (layer Edge.Cuts) (width 0.15))
 (segment (start 161.750 83.219) (end 157.424 89.398) (width 0.2) (layer F.Cu) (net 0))
 (via (at 157.424 89.398) (size 0.6) (drill 0.4) (layers F.Cu B.Cu) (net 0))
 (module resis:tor (layer F.Cu) (at 150 100 55.0)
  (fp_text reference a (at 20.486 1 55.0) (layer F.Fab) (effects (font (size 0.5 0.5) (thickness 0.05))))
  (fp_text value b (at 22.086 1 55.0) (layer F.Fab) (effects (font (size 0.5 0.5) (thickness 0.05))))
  (pad 1 smd rect (at 20.5 0 55.0) (size 0.8 0.8) (layers F.Cu F.Paste F.Mask))
  (pad 2 smd rect (at 22.1 0 55.0) (size 0.8 0.8) (layers F.Cu F.Paste F.Mask)))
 (segment (start 162.668 81.908) (end 163.913 80.130) (width 0.2) (layer F.Cu) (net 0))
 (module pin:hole (layer F.Cu) (at 163.913 80.130)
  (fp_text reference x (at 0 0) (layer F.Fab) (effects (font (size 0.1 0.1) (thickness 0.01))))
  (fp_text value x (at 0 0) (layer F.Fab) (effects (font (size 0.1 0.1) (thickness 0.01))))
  (pad 1 thru_hole rect (at 0 0 55.0) (size 1.7 1.7) (drill 1) (layers *.Cu *.Mask)))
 (gr_line (start 125.000 75.000) (end 125.000 125.000) (angle 90) (layer Edge.Cuts) (width 0.15))
 (gr_line (start 175.000 75.000) (end 175.000 125.000) (angle 90) (layer Edge.Cuts) (width 0.15))
 (gr_line (start 125.000 75.000) (end 175.000 75.000) (angle 0) (layer Edge.Cuts) (width 0.15))
 (gr_line (start 125.000 125.000) (end 175.000 125.000) (angle 0) (layer Edge.Cuts) (width 0.15))
 (segment (start 141.342 81.434) (end 144.132 87.415) (width 0.2) (layer F.Cu) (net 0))
 (via (at 144.132 87.415) (size 0.6) (drill 0.4) (layers F.Cu B.Cu) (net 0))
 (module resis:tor (layer F.Cu) (at 150 100 115.0)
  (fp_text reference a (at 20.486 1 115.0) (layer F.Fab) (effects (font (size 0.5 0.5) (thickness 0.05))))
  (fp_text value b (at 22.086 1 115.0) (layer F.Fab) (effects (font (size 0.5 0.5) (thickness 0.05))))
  (pad 1 smd rect (at 20.5 0 115.0) (size 0.8 0.8) (layers F.Cu F.Paste F.Mask))
  (pad 2 smd rect (at 22.1 0 115.0) (size 0.8 0.8) (layers F.Cu F.Paste F.Mask)))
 (segment (start 140.666 79.984) (end 139.748 78.016) (width 0.2) (layer F.Cu) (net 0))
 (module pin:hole (layer F.Cu) (at 139.748 78.016)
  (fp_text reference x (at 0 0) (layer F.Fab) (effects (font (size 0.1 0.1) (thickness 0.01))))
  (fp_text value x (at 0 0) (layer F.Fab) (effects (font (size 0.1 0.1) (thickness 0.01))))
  (pad 2 thru_hole rect (at 0 0 115.0) (size 1.7 1.7) (drill 1) (layers *.Cu *.Mask)))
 (gr_line (start 125.000 75.000) (end 125.000 125.000) (angle 90) (layer Edge.Cuts) (width 0.15))
 (gr_line (start 175.000 75.000) (end 175.000 125.000) (angle 90) (layer Edge.Cuts) (width 0.15))
 (gr_line (start 125.000 75.000) (end 175.000 75.000) (angle 0) (layer Edge.Cuts) (width 0.15))
 (gr_line (start 125.000 125.000) (end 175.000 125.000) (angle 0) (layer Edge.Cuts) (width 0.15))
 (segment (start 133.219 88.250) (end 137.853 91.495) (width 0.2) (layer F.Cu) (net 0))
 (via (at 137.853 91.495) (size 0.6) (drill 0.4) (layers F.Cu B.Cu) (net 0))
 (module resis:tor (layer F.Cu) (at 150 100 145.0)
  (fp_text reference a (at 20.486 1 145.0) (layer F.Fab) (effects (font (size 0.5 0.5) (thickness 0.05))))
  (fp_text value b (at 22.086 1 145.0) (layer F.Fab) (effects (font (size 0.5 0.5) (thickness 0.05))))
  (pad 1 smd rect (at 20.5 0 145.0) (size 0.8 0.8) (layers F.Cu F.Paste F.Mask))
  (pad 2 smd rect (at 22.1 0 145.0) (size 0.8 0.8) (layers F.Cu F.Paste F.Mask)))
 (segment (start 131.908 87.332) (end 130.130 86.087) (width 0.2) (layer F.Cu) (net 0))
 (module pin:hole (layer F.Cu) (at 130.130 86.087)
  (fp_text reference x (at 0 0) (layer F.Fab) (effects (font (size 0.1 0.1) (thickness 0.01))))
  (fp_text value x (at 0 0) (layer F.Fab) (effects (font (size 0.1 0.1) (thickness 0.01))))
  (pad 3 thru_hole rect (at 0 0 145.0) (size 1.7 1.7) (drill 1) (layers *.Cu *.Mask)))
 (gr_line (start 125.000 75.000) (end 125.000 125.000) (angle 90) (layer Edge.Cuts) (width 0.15))
 (gr_line (start 175.000 75.000) (end 175.000 125.000) (angle 90) (layer Edge.Cuts) (width 0.15))
 (gr_line (start 125.000 75.000) (end 175.000 75.000) (angle 0) (layer Edge.Cuts) (width 0.15))
 (gr_line (start 125.000 125.000) (end 175.000 125.000) (angle 0) (layer Edge.Cuts) (width 0.15))
 (segment (start 131.434 108.658) (end 135.706 106.665) (width 0.2) (layer F.Cu) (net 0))
 (via (at 135.706 106.665) (size 0.6) (drill 0.4) (layers F.Cu B.Cu) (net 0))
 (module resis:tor (layer F.Cu) (at 150 100 205.0)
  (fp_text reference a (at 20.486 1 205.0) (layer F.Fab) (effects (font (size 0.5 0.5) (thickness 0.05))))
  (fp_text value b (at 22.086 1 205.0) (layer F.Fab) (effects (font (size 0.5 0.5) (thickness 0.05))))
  (pad 1 smd rect (at 20.5 0 205.0) (size 0.8 0.8) (layers F.Cu F.Paste F.Mask))
  (pad 2 smd rect (at 22.1 0 205.0) (size 0.8 0.8) (layers F.Cu F.Paste F.Mask)))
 (segment (start 129.984 109.334) (end 128.016 110.252) (width 0.2) (layer F.Cu) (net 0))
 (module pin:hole (layer F.Cu) (at 128.016 110.252)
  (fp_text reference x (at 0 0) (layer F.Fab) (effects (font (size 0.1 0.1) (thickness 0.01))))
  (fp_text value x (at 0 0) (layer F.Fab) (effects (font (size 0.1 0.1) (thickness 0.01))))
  (pad 4 thru_hole rect (at 0 0 205.0) (size 1.7 1.7) (drill 1) (layers *.Cu *.Mask)))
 (gr_line (start 125.000 75.000) (end 125.000 125.000) (angle 90) (layer Edge.Cuts) (width 0.15))
 (gr_line (start 175.000 75.000) (end 175.000 125.000) (angle 90) (layer Edge.Cuts) (width 0.15))
 (gr_line (start 125.000 75.000) (end 175.000 75.000) (angle 0) (layer Edge.Cuts) (width 0.15))
 (gr_line (start 125.000 125.000) (end 175.000 125.000) (angle 0) (layer Edge.Cuts) (width 0.15))
 (segment (start 138.250 116.781) (end 140.413 113.692) (width 0.2) (layer F.Cu) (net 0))
 (via (at 140.413 113.692) (size 0.6) (drill 0.4) (layers F.Cu B.Cu) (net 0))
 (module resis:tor (layer F.Cu) (at 150 100 235.0)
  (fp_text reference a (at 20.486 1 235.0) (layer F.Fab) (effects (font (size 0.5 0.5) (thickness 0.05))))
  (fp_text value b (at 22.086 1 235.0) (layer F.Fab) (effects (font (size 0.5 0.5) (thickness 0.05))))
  (pad 1 smd rect (at 20.5 0 235.0) (size 0.8 0.8) (layers F.Cu F.Paste F.Mask))
  (pad 2 smd rect (at 22.1 0 235.0) (size 0.8 0.8) (layers F.Cu F.Paste F.Mask)))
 (segment (start 137.332 118.092) (end 136.087 119.870) (width 0.2) (layer F.Cu) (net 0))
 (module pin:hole (layer F.Cu) (at 136.087 119.870)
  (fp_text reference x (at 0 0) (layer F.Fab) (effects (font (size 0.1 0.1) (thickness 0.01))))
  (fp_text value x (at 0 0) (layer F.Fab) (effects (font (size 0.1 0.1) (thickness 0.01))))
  (pad 5 thru_hole rect (at 0 0 235.0) (size 1.7 1.7) (drill 1) (layers *.Cu *.Mask)))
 (gr_line (start 125.000 75.000) (end 125.000 125.000) (angle 90) (layer Edge.Cuts) (width 0.15))
 (gr_line (start 175.000 75.000) (end 175.000 125.000) (angle 90) (layer Edge.Cuts) (width 0.15))
 (gr_line (start 125.000 75.000) (end 175.000 75.000) (angle 0) (layer Edge.Cuts) (width 0.15))
 (gr_line (start 125.000 125.000) (end 175.000 125.000) (angle 0) (layer Edge.Cuts) (width 0.15))
 (segment (start 158.658 118.566) (end 157.462 116.003) (width 0.2) (layer F.Cu) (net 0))
 (via (at 157.462 116.003) (size 0.6) (drill 0.4) (layers F.Cu B.Cu) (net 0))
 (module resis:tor (layer F.Cu) (at 150 100 295.0)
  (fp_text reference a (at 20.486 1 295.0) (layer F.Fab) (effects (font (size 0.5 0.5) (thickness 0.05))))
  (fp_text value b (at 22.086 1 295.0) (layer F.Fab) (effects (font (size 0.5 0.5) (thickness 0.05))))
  (pad 1 smd rect (at 20.5 0 295.0) (size 0.8 0.8) (layers F.Cu F.Paste F.Mask))
  (pad 2 smd rect (at 22.1 0 295.0) (size 0.8 0.8) (layers F.Cu F.Paste F.Mask)))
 (segment (start 159.334 120.016) (end 160.252 121.984) (width 0.2) (layer F.Cu) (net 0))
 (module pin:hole (layer F.Cu) (at 160.252 121.984)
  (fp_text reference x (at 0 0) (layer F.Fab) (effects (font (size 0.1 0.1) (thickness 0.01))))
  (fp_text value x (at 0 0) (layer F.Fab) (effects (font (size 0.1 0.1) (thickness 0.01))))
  (pad 6 thru_hole rect (at 0 0 295.0) (size 1.7 1.7) (drill 1) (layers *.Cu *.Mask)))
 (gr_line (start 125.000 75.000) (end 125.000 125.000) (angle 90) (layer Edge.Cuts) (width 0.15))
 (gr_line (start 175.000 75.000) (end 175.000 125.000) (angle 90) (layer Edge.Cuts) (width 0.15))
 (gr_line (start 125.000 75.000) (end 175.000 75.000) (angle 0) (layer Edge.Cuts) (width 0.15))
 (gr_line (start 125.000 125.000) (end 175.000 125.000) (angle 0) (layer Edge.Cuts) (width 0.15))
 (segment (start 166.781 111.750) (end 165.236 110.669) (width 0.2) (layer F.Cu) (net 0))
 (via (at 165.236 110.669) (size 0.6) (drill 0.4) (layers F.Cu B.Cu) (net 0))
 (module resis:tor (layer F.Cu) (at 150 100 325.0)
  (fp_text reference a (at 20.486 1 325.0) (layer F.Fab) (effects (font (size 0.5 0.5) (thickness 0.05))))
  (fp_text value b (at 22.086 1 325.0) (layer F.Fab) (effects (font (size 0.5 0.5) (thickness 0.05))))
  (pad 1 smd rect (at 20.5 0 325.0) (size 0.8 0.8) (layers F.Cu F.Paste F.Mask))
  (pad 2 smd rect (at 22.1 0 325.0) (size 0.8 0.8) (layers F.Cu F.Paste F.Mask)))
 (segment (start 168.092 112.668) (end 169.870 113.913) (width 0.2) (layer F.Cu) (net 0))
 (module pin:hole (layer F.Cu) (at 169.870 113.913)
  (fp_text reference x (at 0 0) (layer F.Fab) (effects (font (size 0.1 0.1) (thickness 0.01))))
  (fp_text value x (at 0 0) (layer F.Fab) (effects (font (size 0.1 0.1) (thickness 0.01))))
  (pad 7 thru_hole rect (at 0 0 325.0) (size 1.7 1.7) (drill 1) (layers *.Cu *.Mask)))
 (gr_line (start 125.000 75.000) (end 125.000 125.000) (angle 90) (layer Edge.Cuts) (width 0.15))
 (gr_line (start 175.000 75.000) (end 175.000 125.000) (angle 90) (layer Edge.Cuts) (width 0.15))
 (gr_line (start 125.000 75.000) (end 175.000 75.000) (angle 0) (layer Edge.Cuts) (width 0.15))
 (gr_line (start 125.000 125.000) (end 175.000 125.000) (angle 0) (layer Edge.Cuts) (width 0.15)))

